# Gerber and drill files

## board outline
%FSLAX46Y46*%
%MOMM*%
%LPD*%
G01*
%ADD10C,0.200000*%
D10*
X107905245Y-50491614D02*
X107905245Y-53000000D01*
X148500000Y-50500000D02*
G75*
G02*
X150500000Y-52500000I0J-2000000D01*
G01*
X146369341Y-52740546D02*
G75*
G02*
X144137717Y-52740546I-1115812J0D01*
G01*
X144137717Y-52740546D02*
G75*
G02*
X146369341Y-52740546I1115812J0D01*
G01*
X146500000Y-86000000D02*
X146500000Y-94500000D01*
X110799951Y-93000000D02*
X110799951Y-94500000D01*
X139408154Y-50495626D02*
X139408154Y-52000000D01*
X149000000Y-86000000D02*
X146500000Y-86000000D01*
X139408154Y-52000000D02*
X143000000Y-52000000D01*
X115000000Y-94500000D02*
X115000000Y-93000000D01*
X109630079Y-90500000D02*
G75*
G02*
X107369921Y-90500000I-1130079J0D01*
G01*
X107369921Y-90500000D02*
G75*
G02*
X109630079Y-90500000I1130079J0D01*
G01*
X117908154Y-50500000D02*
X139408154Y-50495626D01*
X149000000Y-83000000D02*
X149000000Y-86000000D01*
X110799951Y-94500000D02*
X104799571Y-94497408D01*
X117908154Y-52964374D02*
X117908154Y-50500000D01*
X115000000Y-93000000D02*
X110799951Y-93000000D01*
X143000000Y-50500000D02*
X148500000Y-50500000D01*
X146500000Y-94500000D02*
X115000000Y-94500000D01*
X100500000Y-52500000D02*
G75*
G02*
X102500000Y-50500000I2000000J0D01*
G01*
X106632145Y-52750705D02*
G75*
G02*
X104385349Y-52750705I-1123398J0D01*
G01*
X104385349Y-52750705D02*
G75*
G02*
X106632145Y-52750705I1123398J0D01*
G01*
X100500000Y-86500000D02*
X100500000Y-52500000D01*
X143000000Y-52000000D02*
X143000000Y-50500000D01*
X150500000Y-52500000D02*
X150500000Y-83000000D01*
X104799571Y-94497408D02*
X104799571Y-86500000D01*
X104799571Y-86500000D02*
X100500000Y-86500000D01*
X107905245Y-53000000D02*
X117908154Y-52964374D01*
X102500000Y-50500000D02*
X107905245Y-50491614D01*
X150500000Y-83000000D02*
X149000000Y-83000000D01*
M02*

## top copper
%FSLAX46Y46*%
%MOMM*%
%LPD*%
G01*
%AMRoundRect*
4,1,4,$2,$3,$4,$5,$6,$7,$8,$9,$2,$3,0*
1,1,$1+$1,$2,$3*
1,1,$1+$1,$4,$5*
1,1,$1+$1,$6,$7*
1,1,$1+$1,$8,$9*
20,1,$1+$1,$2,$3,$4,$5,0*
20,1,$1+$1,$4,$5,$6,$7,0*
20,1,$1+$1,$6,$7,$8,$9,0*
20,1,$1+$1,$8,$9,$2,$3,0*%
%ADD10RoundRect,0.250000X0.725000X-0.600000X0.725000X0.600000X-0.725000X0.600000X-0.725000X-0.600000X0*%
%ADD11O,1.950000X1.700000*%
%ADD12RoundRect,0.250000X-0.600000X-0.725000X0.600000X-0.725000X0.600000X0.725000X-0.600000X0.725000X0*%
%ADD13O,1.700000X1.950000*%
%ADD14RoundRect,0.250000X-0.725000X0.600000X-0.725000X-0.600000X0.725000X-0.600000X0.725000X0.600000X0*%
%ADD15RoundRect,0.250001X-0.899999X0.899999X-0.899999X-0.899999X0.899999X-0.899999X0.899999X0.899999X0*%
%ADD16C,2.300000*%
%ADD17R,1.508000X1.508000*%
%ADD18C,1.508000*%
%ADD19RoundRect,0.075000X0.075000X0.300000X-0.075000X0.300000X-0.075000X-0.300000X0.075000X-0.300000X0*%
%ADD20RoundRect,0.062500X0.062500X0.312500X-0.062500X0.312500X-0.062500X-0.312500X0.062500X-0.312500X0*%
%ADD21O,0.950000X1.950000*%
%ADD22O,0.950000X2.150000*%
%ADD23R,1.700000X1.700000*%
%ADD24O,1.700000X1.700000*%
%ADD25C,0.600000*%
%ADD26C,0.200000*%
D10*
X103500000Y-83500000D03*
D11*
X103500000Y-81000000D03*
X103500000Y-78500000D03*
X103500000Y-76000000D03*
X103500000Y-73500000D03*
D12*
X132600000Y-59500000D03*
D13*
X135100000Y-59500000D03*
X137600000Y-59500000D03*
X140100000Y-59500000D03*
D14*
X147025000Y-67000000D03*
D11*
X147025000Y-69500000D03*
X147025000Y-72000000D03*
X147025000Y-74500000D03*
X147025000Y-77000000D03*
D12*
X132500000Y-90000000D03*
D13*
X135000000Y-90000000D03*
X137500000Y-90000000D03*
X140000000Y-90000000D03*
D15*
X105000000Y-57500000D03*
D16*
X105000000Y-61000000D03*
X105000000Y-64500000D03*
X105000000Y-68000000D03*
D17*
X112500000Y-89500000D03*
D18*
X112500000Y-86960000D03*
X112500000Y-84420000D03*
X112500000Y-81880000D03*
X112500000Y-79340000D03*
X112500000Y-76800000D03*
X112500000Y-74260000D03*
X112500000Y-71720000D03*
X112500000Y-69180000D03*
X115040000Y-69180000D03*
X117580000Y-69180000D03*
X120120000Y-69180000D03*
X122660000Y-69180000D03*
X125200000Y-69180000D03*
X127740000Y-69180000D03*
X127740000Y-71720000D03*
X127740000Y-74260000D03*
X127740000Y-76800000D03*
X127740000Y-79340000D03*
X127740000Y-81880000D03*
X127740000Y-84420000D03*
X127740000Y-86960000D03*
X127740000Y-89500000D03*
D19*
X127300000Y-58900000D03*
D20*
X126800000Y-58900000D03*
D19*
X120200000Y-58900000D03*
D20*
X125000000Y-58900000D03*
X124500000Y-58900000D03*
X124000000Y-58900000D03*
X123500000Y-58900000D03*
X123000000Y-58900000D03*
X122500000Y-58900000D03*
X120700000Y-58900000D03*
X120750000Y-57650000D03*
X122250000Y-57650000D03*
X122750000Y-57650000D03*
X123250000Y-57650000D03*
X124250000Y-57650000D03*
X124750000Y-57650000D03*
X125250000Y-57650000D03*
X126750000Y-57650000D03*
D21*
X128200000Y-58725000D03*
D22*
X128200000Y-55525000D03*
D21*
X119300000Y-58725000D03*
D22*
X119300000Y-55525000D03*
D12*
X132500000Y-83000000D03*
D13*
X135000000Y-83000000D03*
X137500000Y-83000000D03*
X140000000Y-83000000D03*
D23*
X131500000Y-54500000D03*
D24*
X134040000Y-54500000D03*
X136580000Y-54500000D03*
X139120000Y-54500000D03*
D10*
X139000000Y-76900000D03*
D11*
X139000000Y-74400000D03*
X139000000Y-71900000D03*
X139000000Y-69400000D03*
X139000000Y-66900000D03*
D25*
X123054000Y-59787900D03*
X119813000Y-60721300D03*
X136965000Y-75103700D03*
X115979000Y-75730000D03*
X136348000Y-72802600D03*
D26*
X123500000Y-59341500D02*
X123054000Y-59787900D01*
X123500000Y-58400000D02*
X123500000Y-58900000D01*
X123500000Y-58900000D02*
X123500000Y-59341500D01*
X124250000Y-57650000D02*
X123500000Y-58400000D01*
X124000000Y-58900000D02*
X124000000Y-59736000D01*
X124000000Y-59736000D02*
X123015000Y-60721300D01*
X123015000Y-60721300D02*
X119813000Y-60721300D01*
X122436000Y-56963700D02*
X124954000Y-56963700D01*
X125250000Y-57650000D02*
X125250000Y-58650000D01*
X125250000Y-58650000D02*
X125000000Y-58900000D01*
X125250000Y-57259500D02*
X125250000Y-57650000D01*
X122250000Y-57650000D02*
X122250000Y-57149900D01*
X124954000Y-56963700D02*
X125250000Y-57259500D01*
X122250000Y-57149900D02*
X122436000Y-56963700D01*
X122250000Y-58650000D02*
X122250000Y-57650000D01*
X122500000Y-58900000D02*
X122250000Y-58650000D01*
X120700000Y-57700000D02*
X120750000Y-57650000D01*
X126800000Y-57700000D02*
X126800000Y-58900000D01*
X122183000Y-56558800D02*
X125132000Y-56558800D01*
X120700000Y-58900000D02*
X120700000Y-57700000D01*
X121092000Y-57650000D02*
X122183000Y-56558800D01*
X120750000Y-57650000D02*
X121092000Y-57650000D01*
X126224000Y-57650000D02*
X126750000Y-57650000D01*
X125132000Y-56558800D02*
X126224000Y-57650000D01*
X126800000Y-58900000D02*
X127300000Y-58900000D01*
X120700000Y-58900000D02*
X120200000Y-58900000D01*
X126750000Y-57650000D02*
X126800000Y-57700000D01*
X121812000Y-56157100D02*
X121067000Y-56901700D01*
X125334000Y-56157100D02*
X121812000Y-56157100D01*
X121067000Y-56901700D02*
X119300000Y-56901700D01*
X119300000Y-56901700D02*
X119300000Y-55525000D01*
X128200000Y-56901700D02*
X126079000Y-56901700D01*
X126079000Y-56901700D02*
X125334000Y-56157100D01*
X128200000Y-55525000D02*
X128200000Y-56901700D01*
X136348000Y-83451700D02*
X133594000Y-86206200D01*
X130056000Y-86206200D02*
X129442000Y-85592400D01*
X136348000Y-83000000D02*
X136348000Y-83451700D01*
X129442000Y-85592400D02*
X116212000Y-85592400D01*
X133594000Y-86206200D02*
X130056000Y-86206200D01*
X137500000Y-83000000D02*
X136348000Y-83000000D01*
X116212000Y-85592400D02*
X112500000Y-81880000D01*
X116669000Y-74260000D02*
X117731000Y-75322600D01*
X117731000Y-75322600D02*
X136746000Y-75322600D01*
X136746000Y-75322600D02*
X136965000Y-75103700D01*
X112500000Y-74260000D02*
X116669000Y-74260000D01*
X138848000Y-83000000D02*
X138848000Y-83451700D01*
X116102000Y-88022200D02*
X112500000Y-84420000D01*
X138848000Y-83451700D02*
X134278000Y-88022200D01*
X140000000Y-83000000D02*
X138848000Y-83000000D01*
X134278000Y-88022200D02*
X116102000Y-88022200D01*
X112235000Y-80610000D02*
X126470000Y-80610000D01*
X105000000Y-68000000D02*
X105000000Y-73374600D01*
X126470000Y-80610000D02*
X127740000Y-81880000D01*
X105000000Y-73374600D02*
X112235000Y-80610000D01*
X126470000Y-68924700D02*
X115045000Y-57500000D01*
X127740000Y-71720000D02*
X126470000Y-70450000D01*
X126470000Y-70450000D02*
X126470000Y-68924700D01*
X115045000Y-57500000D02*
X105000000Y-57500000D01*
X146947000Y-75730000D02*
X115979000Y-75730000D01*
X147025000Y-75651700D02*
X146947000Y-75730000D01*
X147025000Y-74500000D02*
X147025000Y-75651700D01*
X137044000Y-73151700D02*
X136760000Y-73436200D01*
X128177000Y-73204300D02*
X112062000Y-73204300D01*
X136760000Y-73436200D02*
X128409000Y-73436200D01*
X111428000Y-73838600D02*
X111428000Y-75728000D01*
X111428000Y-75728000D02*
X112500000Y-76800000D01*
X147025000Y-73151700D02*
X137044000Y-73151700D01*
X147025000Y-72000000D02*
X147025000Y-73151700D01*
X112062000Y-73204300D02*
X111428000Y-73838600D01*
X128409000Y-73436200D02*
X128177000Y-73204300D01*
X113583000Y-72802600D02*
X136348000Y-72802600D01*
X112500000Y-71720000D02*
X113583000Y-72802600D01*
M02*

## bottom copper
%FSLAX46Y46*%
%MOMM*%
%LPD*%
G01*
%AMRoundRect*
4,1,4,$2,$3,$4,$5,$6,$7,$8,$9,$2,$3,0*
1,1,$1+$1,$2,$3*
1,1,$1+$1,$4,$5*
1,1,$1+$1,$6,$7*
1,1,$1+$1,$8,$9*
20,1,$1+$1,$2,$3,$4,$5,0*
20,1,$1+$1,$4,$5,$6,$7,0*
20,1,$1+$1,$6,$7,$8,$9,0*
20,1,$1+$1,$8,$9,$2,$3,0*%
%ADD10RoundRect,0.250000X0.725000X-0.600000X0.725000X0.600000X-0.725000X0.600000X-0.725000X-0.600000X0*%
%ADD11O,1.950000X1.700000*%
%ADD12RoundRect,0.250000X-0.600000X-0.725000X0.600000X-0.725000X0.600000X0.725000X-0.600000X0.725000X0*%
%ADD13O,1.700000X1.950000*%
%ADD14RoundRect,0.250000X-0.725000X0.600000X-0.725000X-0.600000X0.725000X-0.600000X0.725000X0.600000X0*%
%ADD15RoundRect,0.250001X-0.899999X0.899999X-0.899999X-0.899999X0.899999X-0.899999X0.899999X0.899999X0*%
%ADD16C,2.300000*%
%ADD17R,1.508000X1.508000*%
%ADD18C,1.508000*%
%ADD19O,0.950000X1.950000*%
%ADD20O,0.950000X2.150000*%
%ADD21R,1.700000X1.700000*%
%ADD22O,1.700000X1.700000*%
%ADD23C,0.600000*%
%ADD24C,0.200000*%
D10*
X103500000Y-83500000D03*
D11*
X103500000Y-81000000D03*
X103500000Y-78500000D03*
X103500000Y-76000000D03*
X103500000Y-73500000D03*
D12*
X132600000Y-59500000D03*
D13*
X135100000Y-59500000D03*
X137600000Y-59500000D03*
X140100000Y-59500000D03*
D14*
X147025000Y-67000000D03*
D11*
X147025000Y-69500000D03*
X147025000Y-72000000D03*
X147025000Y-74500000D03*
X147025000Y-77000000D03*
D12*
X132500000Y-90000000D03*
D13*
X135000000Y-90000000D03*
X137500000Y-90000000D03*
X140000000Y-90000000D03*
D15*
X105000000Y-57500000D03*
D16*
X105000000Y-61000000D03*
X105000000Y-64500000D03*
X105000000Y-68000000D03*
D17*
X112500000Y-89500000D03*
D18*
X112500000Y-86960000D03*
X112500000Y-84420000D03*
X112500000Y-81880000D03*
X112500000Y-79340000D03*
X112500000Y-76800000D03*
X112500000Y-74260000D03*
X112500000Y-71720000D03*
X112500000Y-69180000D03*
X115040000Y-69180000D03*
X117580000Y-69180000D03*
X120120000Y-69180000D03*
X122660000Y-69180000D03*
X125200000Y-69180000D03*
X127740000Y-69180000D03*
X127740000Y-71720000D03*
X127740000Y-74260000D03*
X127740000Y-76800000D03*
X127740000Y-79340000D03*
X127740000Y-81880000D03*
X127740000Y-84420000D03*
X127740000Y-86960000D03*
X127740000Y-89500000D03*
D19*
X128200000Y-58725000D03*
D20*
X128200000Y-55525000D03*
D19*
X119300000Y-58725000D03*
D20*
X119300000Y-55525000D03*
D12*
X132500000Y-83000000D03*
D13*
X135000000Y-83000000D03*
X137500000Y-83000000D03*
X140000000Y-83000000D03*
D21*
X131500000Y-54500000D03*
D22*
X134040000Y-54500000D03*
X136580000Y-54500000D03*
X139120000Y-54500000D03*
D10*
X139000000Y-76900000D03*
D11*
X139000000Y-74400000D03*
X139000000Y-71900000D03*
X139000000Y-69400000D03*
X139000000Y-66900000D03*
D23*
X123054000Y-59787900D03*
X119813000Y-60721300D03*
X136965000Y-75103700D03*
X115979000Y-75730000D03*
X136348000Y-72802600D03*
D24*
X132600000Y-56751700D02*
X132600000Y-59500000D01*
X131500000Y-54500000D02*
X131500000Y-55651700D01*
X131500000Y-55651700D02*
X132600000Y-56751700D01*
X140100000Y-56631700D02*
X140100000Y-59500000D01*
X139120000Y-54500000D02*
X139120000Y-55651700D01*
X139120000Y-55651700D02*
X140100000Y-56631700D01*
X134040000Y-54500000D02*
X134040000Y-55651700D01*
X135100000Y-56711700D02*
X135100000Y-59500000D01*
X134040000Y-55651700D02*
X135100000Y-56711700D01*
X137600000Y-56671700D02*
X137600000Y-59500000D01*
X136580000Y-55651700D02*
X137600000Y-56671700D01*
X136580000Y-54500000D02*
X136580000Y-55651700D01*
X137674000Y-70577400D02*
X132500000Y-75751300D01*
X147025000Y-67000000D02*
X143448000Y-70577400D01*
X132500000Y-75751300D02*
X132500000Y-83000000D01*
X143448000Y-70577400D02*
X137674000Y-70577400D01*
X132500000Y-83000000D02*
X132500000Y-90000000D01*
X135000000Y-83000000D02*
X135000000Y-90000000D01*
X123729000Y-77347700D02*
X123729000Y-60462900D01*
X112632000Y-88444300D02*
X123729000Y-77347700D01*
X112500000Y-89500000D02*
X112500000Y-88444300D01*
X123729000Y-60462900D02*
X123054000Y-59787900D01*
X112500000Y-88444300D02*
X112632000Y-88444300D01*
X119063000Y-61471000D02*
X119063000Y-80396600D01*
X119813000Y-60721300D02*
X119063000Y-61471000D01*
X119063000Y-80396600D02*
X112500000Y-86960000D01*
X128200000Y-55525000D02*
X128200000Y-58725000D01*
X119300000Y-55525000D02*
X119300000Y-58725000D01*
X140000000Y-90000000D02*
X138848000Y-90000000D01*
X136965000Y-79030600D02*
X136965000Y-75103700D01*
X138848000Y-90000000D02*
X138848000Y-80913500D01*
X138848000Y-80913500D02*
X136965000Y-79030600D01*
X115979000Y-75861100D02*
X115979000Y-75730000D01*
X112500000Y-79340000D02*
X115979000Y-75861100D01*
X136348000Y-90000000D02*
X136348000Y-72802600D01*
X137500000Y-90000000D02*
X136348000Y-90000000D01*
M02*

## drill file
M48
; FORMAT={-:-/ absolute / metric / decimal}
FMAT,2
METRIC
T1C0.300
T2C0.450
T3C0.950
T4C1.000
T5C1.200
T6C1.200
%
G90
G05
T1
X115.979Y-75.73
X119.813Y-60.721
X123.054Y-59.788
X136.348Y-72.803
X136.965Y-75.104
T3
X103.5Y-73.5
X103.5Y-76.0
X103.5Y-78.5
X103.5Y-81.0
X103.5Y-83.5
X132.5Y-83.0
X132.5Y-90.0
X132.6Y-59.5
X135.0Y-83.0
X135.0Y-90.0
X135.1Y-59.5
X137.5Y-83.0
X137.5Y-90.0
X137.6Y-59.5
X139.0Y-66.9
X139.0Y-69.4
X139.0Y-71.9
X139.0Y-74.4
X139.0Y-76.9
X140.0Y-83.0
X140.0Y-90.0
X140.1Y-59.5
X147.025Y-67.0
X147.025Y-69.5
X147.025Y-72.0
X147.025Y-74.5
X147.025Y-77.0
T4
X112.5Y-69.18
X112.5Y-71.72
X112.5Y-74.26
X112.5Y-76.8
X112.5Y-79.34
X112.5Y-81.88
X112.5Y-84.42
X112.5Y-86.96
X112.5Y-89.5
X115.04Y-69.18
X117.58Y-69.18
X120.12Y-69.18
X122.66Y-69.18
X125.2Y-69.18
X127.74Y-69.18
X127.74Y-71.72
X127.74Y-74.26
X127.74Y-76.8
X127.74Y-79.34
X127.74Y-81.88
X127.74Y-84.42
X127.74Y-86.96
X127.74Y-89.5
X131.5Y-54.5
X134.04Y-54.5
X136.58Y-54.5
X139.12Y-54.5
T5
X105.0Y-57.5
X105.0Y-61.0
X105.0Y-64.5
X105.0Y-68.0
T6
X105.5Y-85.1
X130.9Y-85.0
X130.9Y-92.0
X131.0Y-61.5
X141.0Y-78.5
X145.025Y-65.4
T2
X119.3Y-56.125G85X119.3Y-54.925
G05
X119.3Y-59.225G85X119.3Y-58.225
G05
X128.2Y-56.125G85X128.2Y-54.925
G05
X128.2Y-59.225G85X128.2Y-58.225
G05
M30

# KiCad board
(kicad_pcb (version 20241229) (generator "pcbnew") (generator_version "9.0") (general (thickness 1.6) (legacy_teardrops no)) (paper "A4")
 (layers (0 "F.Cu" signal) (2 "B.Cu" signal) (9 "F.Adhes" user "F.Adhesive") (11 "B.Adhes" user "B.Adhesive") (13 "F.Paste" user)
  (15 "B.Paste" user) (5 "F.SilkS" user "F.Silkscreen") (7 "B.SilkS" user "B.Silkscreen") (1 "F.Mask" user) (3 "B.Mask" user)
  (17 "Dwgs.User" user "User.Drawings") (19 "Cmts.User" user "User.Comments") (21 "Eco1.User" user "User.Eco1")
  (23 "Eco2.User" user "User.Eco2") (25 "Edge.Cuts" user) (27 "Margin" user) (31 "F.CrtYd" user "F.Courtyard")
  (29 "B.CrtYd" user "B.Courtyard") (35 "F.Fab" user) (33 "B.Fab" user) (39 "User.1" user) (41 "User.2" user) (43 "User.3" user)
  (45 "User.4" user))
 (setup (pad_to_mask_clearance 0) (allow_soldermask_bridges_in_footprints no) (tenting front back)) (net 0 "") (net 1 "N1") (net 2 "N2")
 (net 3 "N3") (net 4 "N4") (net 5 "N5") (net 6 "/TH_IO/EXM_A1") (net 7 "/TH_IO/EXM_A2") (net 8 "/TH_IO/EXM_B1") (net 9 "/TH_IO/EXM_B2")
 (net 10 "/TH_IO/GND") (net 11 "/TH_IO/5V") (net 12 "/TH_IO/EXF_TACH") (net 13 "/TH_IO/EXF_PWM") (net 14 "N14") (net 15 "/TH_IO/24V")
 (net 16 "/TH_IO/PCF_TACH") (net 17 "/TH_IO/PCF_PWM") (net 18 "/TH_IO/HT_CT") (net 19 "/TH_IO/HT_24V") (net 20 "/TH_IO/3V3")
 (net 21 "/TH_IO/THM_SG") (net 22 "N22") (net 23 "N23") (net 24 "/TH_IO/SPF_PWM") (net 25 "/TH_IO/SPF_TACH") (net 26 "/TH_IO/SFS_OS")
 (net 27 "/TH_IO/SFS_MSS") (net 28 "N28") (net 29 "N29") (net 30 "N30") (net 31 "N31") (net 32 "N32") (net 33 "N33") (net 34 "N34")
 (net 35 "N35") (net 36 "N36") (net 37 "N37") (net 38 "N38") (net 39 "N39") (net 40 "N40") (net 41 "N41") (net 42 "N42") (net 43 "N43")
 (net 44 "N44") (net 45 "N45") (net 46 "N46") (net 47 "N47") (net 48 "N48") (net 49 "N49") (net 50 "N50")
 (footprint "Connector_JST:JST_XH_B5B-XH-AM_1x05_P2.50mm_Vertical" (layer "F.Cu") (at 103.5 83.5 90)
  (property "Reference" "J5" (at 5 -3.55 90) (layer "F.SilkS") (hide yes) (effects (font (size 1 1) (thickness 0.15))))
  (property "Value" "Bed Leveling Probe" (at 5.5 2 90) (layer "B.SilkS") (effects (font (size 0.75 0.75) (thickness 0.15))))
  (pad "" np_thru_hole circle (at -1.6 2 90) (size 1.2 1.2) (drill 1.2) (layers "*.Cu" "*.Mask"))
  (pad "1" thru_hole roundrect (at 0 0 90) (size 1.7 1.95) (drill 0.95) (layers "*.Cu" "*.Mask") (remove_unused_layers no)
   (roundrect_rratio 0.147059) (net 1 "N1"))
  (pad "2" thru_hole oval (at 2.5 0 90) (size 1.7 1.95) (drill 0.95) (layers "*.Cu" "*.Mask") (remove_unused_layers no) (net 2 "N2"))
  (pad "3" thru_hole oval (at 5 0 90) (size 1.7 1.95) (drill 0.95) (layers "*.Cu" "*.Mask") (remove_unused_layers no) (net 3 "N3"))
  (pad "4" thru_hole oval (at 7.5 0 90) (size 1.7 1.95) (drill 0.95) (layers "*.Cu" "*.Mask") (remove_unused_layers no) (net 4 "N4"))
  (pad "5" thru_hole oval (at 10 0 90) (size 1.7 1.95) (drill 0.95) (layers "*.Cu" "*.Mask") (remove_unused_layers no) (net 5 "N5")))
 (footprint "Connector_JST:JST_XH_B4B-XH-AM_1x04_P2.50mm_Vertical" (layer "F.Cu") (at 132.6 59.5)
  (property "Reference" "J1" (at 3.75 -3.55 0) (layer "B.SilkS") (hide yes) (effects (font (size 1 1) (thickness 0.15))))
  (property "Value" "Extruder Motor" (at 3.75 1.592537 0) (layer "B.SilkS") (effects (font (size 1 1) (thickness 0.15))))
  (pad "" np_thru_hole circle (at -1.6 2) (size 1.2 1.2) (drill 1.2) (layers "*.Cu" "*.Mask"))
  (pad "1" thru_hole roundrect (at 0 0) (size 1.7 1.95) (drill 0.95) (layers "*.Cu" "*.Mask") (remove_unused_layers no)
   (roundrect_rratio 0.147059) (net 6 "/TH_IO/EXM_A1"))
  (pad "2" thru_hole oval (at 2.5 0) (size 1.7 1.95) (drill 0.95) (layers "*.Cu" "*.Mask") (remove_unused_layers no) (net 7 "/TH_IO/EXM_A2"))
  (pad "3" thru_hole oval (at 5 0) (size 1.7 1.95) (drill 0.95) (layers "*.Cu" "*.Mask") (remove_unused_layers no) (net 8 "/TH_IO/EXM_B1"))
  (pad "4" thru_hole oval (at 7.5 0) (size 1.7 1.95) (drill 0.95) (layers "*.Cu" "*.Mask") (remove_unused_layers no) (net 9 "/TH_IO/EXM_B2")))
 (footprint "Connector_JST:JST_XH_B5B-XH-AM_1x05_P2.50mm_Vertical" (layer "F.Cu") (at 147.025 67 -90)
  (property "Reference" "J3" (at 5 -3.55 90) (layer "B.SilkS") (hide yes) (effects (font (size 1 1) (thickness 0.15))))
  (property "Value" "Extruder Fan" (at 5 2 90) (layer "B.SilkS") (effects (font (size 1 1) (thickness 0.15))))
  (pad "" np_thru_hole circle (at -1.6 2 270) (size 1.2 1.2) (drill 1.2) (layers "*.Cu" "*.Mask"))
  (pad "1" thru_hole roundrect (at 0 0 270) (size 1.7 1.95) (drill 0.95) (layers "*.Cu" "*.Mask") (remove_unused_layers no)
   (roundrect_rratio 0.147059) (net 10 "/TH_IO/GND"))
  (pad "2" thru_hole oval (at 2.5 0 270) (size 1.7 1.95) (drill 0.95) (layers "*.Cu" "*.Mask") (remove_unused_layers no)
   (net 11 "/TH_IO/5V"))
  (pad "3" thru_hole oval (at 5 0 270) (size 1.7 1.95) (drill 0.95) (layers "*.Cu" "*.Mask") (remove_unused_layers no)
   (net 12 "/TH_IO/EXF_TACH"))
  (pad "4" thru_hole oval (at 7.5 0 270) (size 1.7 1.95) (drill 0.95) (layers "*.Cu" "*.Mask") (remove_unused_layers no)
   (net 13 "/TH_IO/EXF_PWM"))
  (pad "5" thru_hole oval (at 10 0 270) (size 1.7 1.95) (drill 0.95) (layers "*.Cu" "*.Mask") (remove_unused_layers no) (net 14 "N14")))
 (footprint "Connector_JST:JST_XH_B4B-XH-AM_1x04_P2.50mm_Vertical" (layer "F.Cu") (at 132.5 90)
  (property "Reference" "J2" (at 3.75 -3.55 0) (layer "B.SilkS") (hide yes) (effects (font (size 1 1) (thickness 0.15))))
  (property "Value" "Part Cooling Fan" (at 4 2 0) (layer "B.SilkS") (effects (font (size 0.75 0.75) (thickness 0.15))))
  (pad "" np_thru_hole circle (at -1.6 2) (size 1.2 1.2) (drill 1.2) (layers "*.Cu" "*.Mask"))
  (pad "1" thru_hole roundrect (at 0 0) (size 1.7 1.95) (drill 0.95) (layers "*.Cu" "*.Mask") (remove_unused_layers no)
   (roundrect_rratio 0.147059) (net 10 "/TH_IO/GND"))
  (pad "2" thru_hole oval (at 2.5 0) (size 1.7 1.95) (drill 0.95) (layers "*.Cu" "*.Mask") (remove_unused_layers no) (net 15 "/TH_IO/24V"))
  (pad "3" thru_hole oval (at 5 0) (size 1.7 1.95) (drill 0.95) (layers "*.Cu" "*.Mask") (remove_unused_layers no)
   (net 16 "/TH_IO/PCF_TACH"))
  (pad "4" thru_hole oval (at 7.5 0) (size 1.7 1.95) (drill 0.95) (layers "*.Cu" "*.Mask") (remove_unused_layers no)
   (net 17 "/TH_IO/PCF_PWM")))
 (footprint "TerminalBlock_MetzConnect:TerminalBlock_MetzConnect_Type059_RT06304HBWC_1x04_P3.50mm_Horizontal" (layer "F.Cu")
  (at 105 57.5 -90)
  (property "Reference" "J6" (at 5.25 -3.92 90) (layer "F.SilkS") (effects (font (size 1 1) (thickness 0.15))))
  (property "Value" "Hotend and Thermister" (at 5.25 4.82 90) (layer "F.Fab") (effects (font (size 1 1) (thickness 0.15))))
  (pad "1" thru_hole roundrect (at 0 0 270) (size 2.3 2.3) (drill 1.2) (layers "*.Cu" "*.Mask") (remove_unused_layers no)
   (roundrect_rratio 0.108696) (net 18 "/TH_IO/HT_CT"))
  (pad "2" thru_hole circle (at 3.5 0 270) (size 2.3 2.3) (drill 1.2) (layers "*.Cu" "*.Mask") (remove_unused_layers no)
   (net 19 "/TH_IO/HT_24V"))
  (pad "3" thru_hole circle (at 7 0 270) (size 2.3 2.3) (drill 1.2) (layers "*.Cu" "*.Mask") (remove_unused_layers no) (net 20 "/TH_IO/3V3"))
  (pad "4" thru_hole circle (at 10.5 0 270) (size 2.3 2.3) (drill 1.2) (layers "*.Cu" "*.Mask") (remove_unused_layers no)
   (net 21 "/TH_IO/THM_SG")))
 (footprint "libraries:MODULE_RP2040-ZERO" (layer "F.Cu") (at 120.12 79.34 180)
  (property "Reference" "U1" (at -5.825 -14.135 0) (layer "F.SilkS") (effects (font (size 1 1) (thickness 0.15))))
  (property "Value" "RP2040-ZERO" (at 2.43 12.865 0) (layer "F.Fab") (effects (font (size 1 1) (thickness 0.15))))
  (pad "1" thru_hole rect (at 7.62 -10.16 180) (size 1.508 1.508) (drill 1) (layers "*.Cu" "*.Mask") (remove_unused_layers no)
   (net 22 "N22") (solder_mask_margin 0.102))
  (pad "2" thru_hole circle (at 7.62 -7.62 180) (size 1.508 1.508) (drill 1) (layers "*.Cu" "*.Mask") (remove_unused_layers no)
   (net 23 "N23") (solder_mask_margin 0.102))
  (pad "3" thru_hole circle (at 7.62 -5.08 180) (size 1.508 1.508) (drill 1) (layers "*.Cu" "*.Mask") (remove_unused_layers no)
   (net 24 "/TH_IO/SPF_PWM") (solder_mask_margin 0.102))
  (pad "4" thru_hole circle (at 7.62 -2.54 180) (size 1.508 1.508) (drill 1) (layers "*.Cu" "*.Mask") (remove_unused_layers no)
   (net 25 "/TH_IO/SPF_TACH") (solder_mask_margin 0.102))
  (pad "5" thru_hole circle (at 7.62 0 180) (size 1.508 1.508) (drill 1) (layers "*.Cu" "*.Mask") (remove_unused_layers no)
   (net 13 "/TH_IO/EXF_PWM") (solder_mask_margin 0.102))
  (pad "6" thru_hole circle (at 7.62 2.54 180) (size 1.508 1.508) (drill 1) (layers "*.Cu" "*.Mask") (remove_unused_layers no)
   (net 12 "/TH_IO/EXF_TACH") (solder_mask_margin 0.102))
  (pad "7" thru_hole circle (at 7.62 5.08 180) (size 1.508 1.508) (drill 1) (layers "*.Cu" "*.Mask") (remove_unused_layers no)
   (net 17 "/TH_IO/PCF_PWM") (solder_mask_margin 0.102))
  (pad "8" thru_hole circle (at 7.62 7.62 180) (size 1.508 1.508) (drill 1) (layers "*.Cu" "*.Mask") (remove_unused_layers no)
   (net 16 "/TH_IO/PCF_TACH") (solder_mask_margin 0.102))
  (pad "9" thru_hole circle (at 7.62 10.16 180) (size 1.508 1.508) (drill 1) (layers "*.Cu" "*.Mask") (remove_unused_layers no)
   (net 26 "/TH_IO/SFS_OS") (solder_mask_margin 0.102))
  (pad "10" thru_hole circle (at 5.08 10.16 180) (size 1.508 1.508) (drill 1) (layers "*.Cu" "*.Mask") (remove_unused_layers no)
   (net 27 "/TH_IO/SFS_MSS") (solder_mask_margin 0.102))
  (pad "11" thru_hole circle (at 2.54 10.16 180) (size 1.508 1.508) (drill 1) (layers "*.Cu" "*.Mask") (remove_unused_layers no)
   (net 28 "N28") (solder_mask_margin 0.102))
  (pad "12" thru_hole circle (at 0 10.16 180) (size 1.508 1.508) (drill 1) (layers "*.Cu" "*.Mask") (remove_unused_layers no) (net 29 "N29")
   (solder_mask_margin 0.102))
  (pad "13" thru_hole circle (at -2.54 10.16 180) (size 1.508 1.508) (drill 1) (layers "*.Cu" "*.Mask") (remove_unused_layers no)
   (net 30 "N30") (solder_mask_margin 0.102))
  (pad "14" thru_hole circle (at -5.08 10.16 180) (size 1.508 1.508) (drill 1) (layers "*.Cu" "*.Mask") (remove_unused_layers no)
   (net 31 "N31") (solder_mask_margin 0.102))
  (pad "15" thru_hole circle (at -7.62 10.16 180) (size 1.508 1.508) (drill 1) (layers "*.Cu" "*.Mask") (remove_unused_layers no)
   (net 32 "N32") (solder_mask_margin 0.102))
  (pad "16" thru_hole circle (at -7.62 7.62 180) (size 1.508 1.508) (drill 1) (layers "*.Cu" "*.Mask") (remove_unused_layers no)
   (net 18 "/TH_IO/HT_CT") (solder_mask_margin 0.102))
  (pad "17" thru_hole circle (at -7.62 5.08 180) (size 1.508 1.508) (drill 1) (layers "*.Cu" "*.Mask") (remove_unused_layers no)
   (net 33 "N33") (solder_mask_margin 0.102))
  (pad "18" thru_hole circle (at -7.62 2.54 180) (size 1.508 1.508) (drill 1) (layers "*.Cu" "*.Mask") (remove_unused_layers no)
   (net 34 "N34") (solder_mask_margin 0.102))
  (pad "19" thru_hole circle (at -7.62 0 180) (size 1.508 1.508) (drill 1) (layers "*.Cu" "*.Mask") (remove_unused_layers no) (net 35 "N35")
   (solder_mask_margin 0.102))
  (pad "20" thru_hole circle (at -7.62 -2.54 180) (size 1.508 1.508) (drill 1) (layers "*.Cu" "*.Mask") (remove_unused_layers no)
   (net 21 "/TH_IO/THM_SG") (solder_mask_margin 0.102))
  (pad "21" thru_hole circle (at -7.62 -5.08 180) (size 1.508 1.508) (drill 1) (layers "*.Cu" "*.Mask") (remove_unused_layers no)
   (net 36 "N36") (solder_mask_margin 0.102))
  (pad "22" thru_hole circle (at -7.62 -7.62 180) (size 1.508 1.508) (drill 1) (layers "*.Cu" "*.Mask") (remove_unused_layers no)
   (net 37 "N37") (solder_mask_margin 0.102))
  (pad "23" thru_hole circle (at -7.62 -10.16 180) (size 1.508 1.508) (drill 1) (layers "*.Cu" "*.Mask") (remove_unused_layers no)
   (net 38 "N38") (solder_mask_margin 0.102)))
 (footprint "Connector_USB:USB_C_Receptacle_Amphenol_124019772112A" (layer "F.Cu") (at 123.75 55.7 180)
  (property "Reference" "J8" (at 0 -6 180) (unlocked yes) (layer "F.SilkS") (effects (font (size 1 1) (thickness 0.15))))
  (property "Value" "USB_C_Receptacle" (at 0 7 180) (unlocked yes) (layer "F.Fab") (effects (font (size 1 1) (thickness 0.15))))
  (pad "A1" smd roundrect (at -3.55 -3.2 180) (size 0.3 0.75) (layers "F.Cu" "F.Mask" "F.Paste") (roundrect_rratio 0.25) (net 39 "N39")
   (thermal_bridge_angle 45))
  (pad "A1" smd roundrect (at -3.05 -3.2 180) (size 0.25 0.75) (layers "F.Cu" "F.Mask" "F.Paste") (roundrect_rratio 0.25) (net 39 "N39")
   (thermal_bridge_angle 45))
  (pad "A1" smd roundrect (at 3.55 -3.2 180) (size 0.3 0.75) (layers "F.Cu" "F.Mask" "F.Paste") (roundrect_rratio 0.25) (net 39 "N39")
   (thermal_bridge_angle 45))
  (pad "A4" smd roundrect (at -1.25 -3.2 180) (size 0.25 0.75) (layers "F.Cu" "F.Mask" "F.Paste") (roundrect_rratio 0.25) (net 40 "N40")
   (thermal_bridge_angle 45))
  (pad "A5" smd roundrect (at -0.75 -3.2 180) (size 0.25 0.75) (layers "F.Cu" "F.Mask" "F.Paste") (roundrect_rratio 0.25) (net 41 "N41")
   (thermal_bridge_angle 45))
  (pad "A6" smd roundrect (at -0.25 -3.2 180) (size 0.25 0.75) (layers "F.Cu" "F.Mask" "F.Paste") (roundrect_rratio 0.25) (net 23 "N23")
   (thermal_bridge_angle 45))
  (pad "A7" smd roundrect (at 0.25 -3.2 180) (size 0.25 0.75) (layers "F.Cu" "F.Mask" "F.Paste") (roundrect_rratio 0.25) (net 22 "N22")
   (thermal_bridge_angle 45))
  (pad "A8" smd roundrect (at 0.75 -3.2 180) (size 0.25 0.75) (layers "F.Cu" "F.Mask" "F.Paste") (roundrect_rratio 0.25) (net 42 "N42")
   (thermal_bridge_angle 45))
  (pad "A9" smd roundrect (at 1.25 -3.2 180) (size 0.25 0.75) (layers "F.Cu" "F.Mask" "F.Paste") (roundrect_rratio 0.25) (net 40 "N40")
   (thermal_bridge_angle 45))
  (pad "A12" smd roundrect (at 3.05 -3.2 180) (size 0.25 0.75) (layers "F.Cu" "F.Mask" "F.Paste") (roundrect_rratio 0.25) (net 39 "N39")
   (thermal_bridge_angle 45))
  (pad "B1" smd roundrect (at 3 -1.95 180) (size 0.25 0.75) (layers "F.Cu" "F.Mask" "F.Paste") (roundrect_rratio 0.25) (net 39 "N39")
   (thermal_bridge_angle 45))
  (pad "B4" smd roundrect (at 1.5 -1.95 180) (size 0.25 0.75) (layers "F.Cu" "F.Mask" "F.Paste") (roundrect_rratio 0.25) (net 40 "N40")
   (thermal_bridge_angle 45))
  (pad "B5" smd roundrect (at 1 -1.95 180) (size 0.25 0.75) (layers "F.Cu" "F.Mask" "F.Paste") (roundrect_rratio 0.25) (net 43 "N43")
   (thermal_bridge_angle 45))
  (pad "B6" smd roundrect (at 0.5 -1.95 180) (size 0.25 0.75) (layers "F.Cu" "F.Mask" "F.Paste") (roundrect_rratio 0.25) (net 23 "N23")
   (thermal_bridge_angle 45))
  (pad "B7" smd roundrect (at -0.5 -1.95 180) (size 0.25 0.75) (layers "F.Cu" "F.Mask" "F.Paste") (roundrect_rratio 0.25) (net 22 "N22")
   (thermal_bridge_angle 45))
  (pad "B8" smd roundrect (at -1 -1.95 180) (size 0.25 0.75) (layers "F.Cu" "F.Mask" "F.Paste") (roundrect_rratio 0.25) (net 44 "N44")
   (thermal_bridge_angle 45))
  (pad "B9" smd roundrect (at -1.5 -1.95 180) (size 0.25 0.75) (layers "F.Cu" "F.Mask" "F.Paste") (roundrect_rratio 0.25) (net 40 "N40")
   (thermal_bridge_angle 45))
  (pad "B12" smd roundrect (at -3 -1.95 180) (size 0.25 0.75) (layers "F.Cu" "F.Mask" "F.Paste") (roundrect_rratio 0.25) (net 39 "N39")
   (thermal_bridge_angle 45))
  (pad "S1" thru_hole oval (at -4.45 -3.025 180) (size 0.95 1.95) (drill oval 0.45 1.45) (layers "*.Cu" "*.Mask") (remove_unused_layers no)
   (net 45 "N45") (thermal_bridge_angle 45))
  (pad "S1" thru_hole oval (at -4.45 0.175 180) (size 0.95 2.15) (drill oval 0.45 1.65) (layers "*.Cu" "*.Mask") (remove_unused_layers no)
   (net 45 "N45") (thermal_bridge_angle 45))
  (pad "S1" thru_hole oval (at 4.45 -3.025 180) (size 0.95 1.95) (drill oval 0.45 1.45) (layers "*.Cu" "*.Mask") (remove_unused_layers no)
   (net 45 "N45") (thermal_bridge_angle 45))
  (pad "S1" thru_hole oval (at 4.45 0.175 180) (size 0.95 2.15) (drill oval 0.45 1.65) (layers "*.Cu" "*.Mask") (remove_unused_layers no)
   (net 45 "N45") (thermal_bridge_angle 45)))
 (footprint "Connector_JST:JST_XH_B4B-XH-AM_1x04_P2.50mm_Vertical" (layer "F.Cu") (at 132.5 83)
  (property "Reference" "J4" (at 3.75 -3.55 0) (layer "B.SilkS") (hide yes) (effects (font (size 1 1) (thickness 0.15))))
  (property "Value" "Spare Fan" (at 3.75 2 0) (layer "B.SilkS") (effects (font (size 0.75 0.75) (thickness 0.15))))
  (pad "" np_thru_hole circle (at -1.6 2) (size 1.2 1.2) (drill 1.2) (layers "*.Cu" "*.Mask"))
  (pad "1" thru_hole roundrect (at 0 0) (size 1.7 1.95) (drill 0.95) (layers "*.Cu" "*.Mask") (remove_unused_layers no)
   (roundrect_rratio 0.147059) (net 10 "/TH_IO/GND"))
  (pad "2" thru_hole oval (at 2.5 0) (size 1.7 1.95) (drill 0.95) (layers "*.Cu" "*.Mask") (remove_unused_layers no) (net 15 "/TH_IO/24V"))
  (pad "3" thru_hole oval (at 5 0) (size 1.7 1.95) (drill 0.95) (layers "*.Cu" "*.Mask") (remove_unused_layers no)
   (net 25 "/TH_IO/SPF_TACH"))
  (pad "4" thru_hole oval (at 7.5 0) (size 1.7 1.95) (drill 0.95) (layers "*.Cu" "*.Mask") (remove_unused_layers no)
   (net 24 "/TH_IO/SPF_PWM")))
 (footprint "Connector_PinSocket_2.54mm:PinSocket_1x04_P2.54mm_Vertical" (layer "F.Cu") (at 131.5 54.5 90)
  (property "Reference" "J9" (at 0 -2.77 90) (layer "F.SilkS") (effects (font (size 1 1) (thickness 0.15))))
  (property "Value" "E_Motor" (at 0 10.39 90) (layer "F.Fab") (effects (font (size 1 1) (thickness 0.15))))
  (pad "1" thru_hole rect (at 0 0 90) (size 1.7 1.7) (drill 1) (layers "*.Cu" "*.Mask") (remove_unused_layers no) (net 6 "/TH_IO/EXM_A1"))
  (pad "2" thru_hole oval (at 0 2.54 90) (size 1.7 1.7) (drill 1) (layers "*.Cu" "*.Mask") (remove_unused_layers no) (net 7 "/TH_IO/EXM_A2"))
  (pad "3" thru_hole oval (at 0 5.08 90) (size 1.7 1.7) (drill 1) (layers "*.Cu" "*.Mask") (remove_unused_layers no) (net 8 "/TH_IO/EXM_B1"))
  (pad "4" thru_hole oval (at 0 7.62 90) (size 1.7 1.7) (drill 1) (layers "*.Cu" "*.Mask") (remove_unused_layers no) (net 9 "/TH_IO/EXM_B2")))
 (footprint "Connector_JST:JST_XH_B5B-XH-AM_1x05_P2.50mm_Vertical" (layer "F.Cu") (at 139 76.9 90)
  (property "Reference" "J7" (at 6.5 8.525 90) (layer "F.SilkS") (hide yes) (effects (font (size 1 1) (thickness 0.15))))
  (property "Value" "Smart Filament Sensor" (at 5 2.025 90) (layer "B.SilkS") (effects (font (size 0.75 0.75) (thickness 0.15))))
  (pad "" np_thru_hole circle (at -1.6 2 90) (size 1.2 1.2) (drill 1.2) (layers "*.Cu" "*.Mask"))
  (pad "1" thru_hole roundrect (at 0 0 90) (size 1.7 1.95) (drill 0.95) (layers "*.Cu" "*.Mask") (remove_unused_layers no)
   (roundrect_rratio 0.147059) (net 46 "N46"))
  (pad "2" thru_hole oval (at 2.5 0 90) (size 1.7 1.95) (drill 0.95) (layers "*.Cu" "*.Mask") (remove_unused_layers no) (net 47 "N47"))
  (pad "3" thru_hole oval (at 5 0 90) (size 1.7 1.95) (drill 0.95) (layers "*.Cu" "*.Mask") (remove_unused_layers no) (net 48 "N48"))
  (pad "4" thru_hole oval (at 7.5 0 90) (size 1.7 1.95) (drill 0.95) (layers "*.Cu" "*.Mask") (remove_unused_layers no) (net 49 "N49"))
  (pad "5" thru_hole oval (at 10 0 90) (size 1.7 1.95) (drill 0.95) (layers "*.Cu" "*.Mask") (remove_unused_layers no) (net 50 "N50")))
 (gr_line (start 107.905245 50.491614) (end 107.905245 53) (stroke (width 0.2) (type solid)) (layer "Edge.Cuts"))
 (gr_arc (start 148.5 50.5) (mid 149.914214 51.085786) (end 150.5 52.5) (stroke (width 0.2) (type solid)) (layer "Edge.Cuts"))
 (gr_circle (center 145.253529 52.740546) (end 144.138266 52.775535) (stroke (width 0.2) (type solid)) (fill no) (layer "Edge.Cuts"))
 (gr_line (start 146.5 86) (end 146.5 94.5) (stroke (width 0.2) (type solid)) (layer "Edge.Cuts"))
 (gr_line (start 110.799951 93) (end 110.799951 94.5) (stroke (width 0.2) (type solid)) (layer "Edge.Cuts"))
 (gr_line (start 139.408154 50.495626) (end 139.408154 52) (stroke (width 0.2) (type solid)) (layer "Edge.Cuts"))
 (gr_line (start 149 86) (end 146.5 86) (stroke (width 0.2) (type solid)) (layer "Edge.Cuts"))
 (gr_line (start 139.408154 52) (end 143 52) (stroke (width 0.2) (type solid)) (layer "Edge.Cuts"))
 (gr_line (start 115 94.5) (end 115 93) (stroke (width 0.2) (type solid)) (layer "Edge.Cuts"))
 (gr_circle (center 108.5 90.5) (end 107.370204 90.474714) (stroke (width 0.2) (type solid)) (fill no) (layer "Edge.Cuts"))
 (gr_line (start 117.908154 50.5) (end 139.408154 50.495626) (stroke (width 0.2) (type solid)) (layer "Edge.Cuts"))
 (gr_line (start 149 83) (end 149 86) (stroke (width 0.2) (type solid)) (layer "Edge.Cuts"))
 (gr_line (start 110.799951 94.5) (end 104.799571 94.497408) (stroke (width 0.2) (type solid)) (layer "Edge.Cuts"))
 (gr_line (start 117.908154 52.964374) (end 117.908154 50.5) (stroke (width 0.2) (type solid)) (layer "Edge.Cuts"))
 (gr_line (start 115 93) (end 110.799951 93) (stroke (width 0.2) (type solid)) (layer "Edge.Cuts"))
 (gr_line (start 143 50.5) (end 148.5 50.5) (stroke (width 0.2) (type solid)) (layer "Edge.Cuts"))
 (gr_line (start 146.5 94.5) (end 115 94.5) (stroke (width 0.2) (type solid)) (layer "Edge.Cuts"))
 (gr_arc (start 100.5 52.5) (mid 101.085786 51.085786) (end 102.5 50.5) (stroke (width 0.2) (type solid)) (layer "Edge.Cuts"))
 (gr_circle (center 105.508747 52.750705) (end 104.38911 52.842551) (stroke (width 0.2) (type solid)) (fill no) (layer "Edge.Cuts"))
 (gr_line (start 100.5 86.5) (end 100.5 52.5) (stroke (width 0.2) (type solid)) (layer "Edge.Cuts"))
 (gr_line (start 143 52) (end 143 50.5) (stroke (width 0.2) (type solid)) (layer "Edge.Cuts"))
 (gr_line (start 150.5 52.5) (end 150.5 83) (stroke (width 0.2) (type solid)) (layer "Edge.Cuts"))
 (gr_line (start 104.799571 94.497408) (end 104.799571 86.5) (stroke (width 0.2) (type solid)) (layer "Edge.Cuts"))
 (gr_line (start 104.799571 86.5) (end 100.5 86.5) (stroke (width 0.2) (type solid)) (layer "Edge.Cuts"))
 (gr_line (start 107.905245 53) (end 117.908154 52.964374) (stroke (width 0.2) (type solid)) (layer "Edge.Cuts"))
 (gr_line (start 102.5 50.5) (end 107.905245 50.491614) (stroke (width 0.2) (type solid)) (layer "Edge.Cuts"))
 (gr_line (start 150.5 83) (end 149 83) (stroke (width 0.2) (type solid)) (layer "Edge.Cuts"))
 (segment (start 132.6 56.7517) (end 132.6 59.5) (width 0.2) (layer "B.Cu") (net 6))
 (segment (start 131.5 54.5) (end 131.5 55.6517) (width 0.2) (layer "B.Cu") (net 6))
 (segment (start 131.5 55.6517) (end 132.6 56.7517) (width 0.2) (layer "B.Cu") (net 6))
 (segment (start 140.1 56.6317) (end 140.1 59.5) (width 0.2) (layer "B.Cu") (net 9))
 (segment (start 139.12 54.5) (end 139.12 55.6517) (width 0.2) (layer "B.Cu") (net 9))
 (segment (start 139.12 55.6517) (end 140.1 56.6317) (width 0.2) (layer "B.Cu") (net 9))
 (segment (start 134.04 54.5) (end 134.04 55.6517) (width 0.2) (layer "B.Cu") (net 7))
 (segment (start 135.1 56.7117) (end 135.1 59.5) (width 0.2) (layer "B.Cu") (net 7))
 (segment (start 134.04 55.6517) (end 135.1 56.7117) (width 0.2) (layer "B.Cu") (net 7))
 (segment (start 137.6 56.6717) (end 137.6 59.5) (width 0.2) (layer "B.Cu") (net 8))
 (segment (start 136.58 55.6517) (end 137.6 56.6717) (width 0.2) (layer "B.Cu") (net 8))
 (segment (start 136.58 54.5) (end 136.58 55.6517) (width 0.2) (layer "B.Cu") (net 8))
 (segment (start 137.674 70.5774) (end 132.5 75.7513) (width 0.2) (layer "B.Cu") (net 10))
 (segment (start 147.025 67) (end 143.448 70.5774) (width 0.2) (layer "B.Cu") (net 10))
 (segment (start 132.5 75.7513) (end 132.5 83) (width 0.2) (layer "B.Cu") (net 10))
 (segment (start 143.448 70.5774) (end 137.674 70.5774) (width 0.2) (layer "B.Cu") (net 10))
 (segment (start 132.5 83) (end 132.5 90) (width 0.2) (layer "B.Cu") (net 10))
 (segment (start 135 83) (end 135 90) (width 0.2) (layer "B.Cu") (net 15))
 (segment (start 123.5 59.3415) (end 123.054 59.7879) (width 0.2) (layer "F.Cu") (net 22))
 (segment (start 123.5 58.4) (end 123.5 58.9) (width 0.2) (layer "F.Cu") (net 22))
 (segment (start 123.5 58.9) (end 123.5 59.3415) (width 0.2) (layer "F.Cu") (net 22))
 (segment (start 124.25 57.65) (end 123.5 58.4) (width 0.2) (layer "F.Cu") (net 22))
 (via (at 123.054 59.7879) (size 0.6) (drill 0.3) (layers "F.Cu" "B.Cu") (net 22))
 (segment (start 123.729 77.3477) (end 123.729 60.4629) (width 0.2) (layer "B.Cu") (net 22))
 (segment (start 112.632 88.4443) (end 123.729 77.3477) (width 0.2) (layer "B.Cu") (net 22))
 (segment (start 112.5 89.5) (end 112.5 88.4443) (width 0.2) (layer "B.Cu") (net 22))
 (segment (start 123.729 60.4629) (end 123.054 59.7879) (width 0.2) (layer "B.Cu") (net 22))
 (segment (start 112.5 88.4443) (end 112.632 88.4443) (width 0.2) (layer "B.Cu") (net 22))
 (segment (start 124 58.9) (end 124 59.736) (width 0.2) (layer "F.Cu") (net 23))
 (segment (start 124 59.736) (end 123.015 60.7213) (width 0.2) (layer "F.Cu") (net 23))
 (segment (start 123.015 60.7213) (end 119.813 60.7213) (width 0.2) (layer "F.Cu") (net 23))
 (via (at 119.813 60.7213) (size 0.6) (drill 0.3) (layers "F.Cu" "B.Cu") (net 23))
 (segment (start 119.063 61.471) (end 119.063 80.3966) (width 0.2) (layer "B.Cu") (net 23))
 (segment (start 119.813 60.7213) (end 119.063 61.471) (width 0.2) (layer "B.Cu") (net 23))
 (segment (start 119.063 80.3966) (end 112.5 86.96) (width 0.2) (layer "B.Cu") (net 23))
 (segment (start 122.436 56.9637) (end 124.954 56.9637) (width 0.2) (layer "F.Cu") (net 40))
 (segment (start 125.25 57.65) (end 125.25 58.65) (width 0.2) (layer "F.Cu") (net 40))
 (segment (start 125.25 58.65) (end 125 58.9) (width 0.2) (layer "F.Cu") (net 40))
 (segment (start 125.25 57.2595) (end 125.25 57.65) (width 0.2) (layer "F.Cu") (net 40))
 (segment (start 122.25 57.65) (end 122.25 57.1499) (width 0.2) (layer "F.Cu") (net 40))
 (segment (start 124.954 56.9637) (end 125.25 57.2595) (width 0.2) (layer "F.Cu") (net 40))
 (segment (start 122.25 57.1499) (end 122.436 56.9637) (width 0.2) (layer "F.Cu") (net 40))
 (segment (start 122.25 58.65) (end 122.25 57.65) (width 0.2) (layer "F.Cu") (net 40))
 (segment (start 122.5 58.9) (end 122.25 58.65) (width 0.2) (layer "F.Cu") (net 40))
 (segment (start 120.7 57.7) (end 120.75 57.65) (width 0.2) (layer "F.Cu") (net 39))
 (segment (start 126.8 57.7) (end 126.8 58.9) (width 0.2) (layer "F.Cu") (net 39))
 (segment (start 122.183 56.5588) (end 125.132 56.5588) (width 0.2) (layer "F.Cu") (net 39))
 (segment (start 120.7 58.9) (end 120.7 57.7) (width 0.2) (layer "F.Cu") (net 39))
 (segment (start 121.092 57.65) (end 122.183 56.5588) (width 0.2) (layer "F.Cu") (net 39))
 (segment (start 120.75 57.65) (end 121.092 57.65) (width 0.2) (layer "F.Cu") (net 39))
 (segment (start 126.224 57.65) (end 126.75 57.65) (width 0.2) (layer "F.Cu") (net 39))
 (segment (start 125.132 56.5588) (end 126.224 57.65) (width 0.2) (layer "F.Cu") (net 39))
 (segment (start 126.8 58.9) (end 127.3 58.9) (width 0.2) (layer "F.Cu") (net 39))
 (segment (start 120.7 58.9) (end 120.2 58.9) (width 0.2) (layer "F.Cu") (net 39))
 (segment (start 126.75 57.65) (end 126.8 57.7) (width 0.2) (layer "F.Cu") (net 39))
 (segment (start 121.812 56.1571) (end 121.067 56.9017) (width 0.2) (layer "F.Cu") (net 45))
 (segment (start 125.334 56.1571) (end 121.812 56.1571) (width 0.2) (layer "F.Cu") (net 45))
 (segment (start 121.067 56.9017) (end 119.3 56.9017) (width 0.2) (layer "F.Cu") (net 45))
 (segment (start 119.3 56.9017) (end 119.3 55.525) (width 0.2) (layer "F.Cu") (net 45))
 (segment (start 128.2 56.9017) (end 126.079 56.9017) (width 0.2) (layer "F.Cu") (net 45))
 (segment (start 126.079 56.9017) (end 125.334 56.1571) (width 0.2) (layer "F.Cu") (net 45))
 (segment (start 128.2 55.525) (end 128.2 56.9017) (width 0.2) (layer "F.Cu") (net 45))
 (segment (start 128.2 55.525) (end 128.2 58.725) (width 0.2) (layer "B.Cu") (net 45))
 (segment (start 119.3 55.525) (end 119.3 58.725) (width 0.2) (layer "B.Cu") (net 45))
 (segment (start 136.348 83.4517) (end 133.594 86.2062) (width 0.2) (layer "F.Cu") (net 25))
 (segment (start 130.056 86.2062) (end 129.442 85.5924) (width 0.2) (layer "F.Cu") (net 25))
 (segment (start 136.348 83) (end 136.348 83.4517) (width 0.2) (layer "F.Cu") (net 25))
 (segment (start 129.442 85.5924) (end 116.212 85.5924) (width 0.2) (layer "F.Cu") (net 25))
 (segment (start 133.594 86.2062) (end 130.056 86.2062) (width 0.2) (layer "F.Cu") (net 25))
 (segment (start 137.5 83) (end 136.348 83) (width 0.2) (layer "F.Cu") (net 25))
 (segment (start 116.212 85.5924) (end 112.5 81.88) (width 0.2) (layer "F.Cu") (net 25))
 (segment (start 116.669 74.26) (end 117.731 75.3226) (width 0.2) (layer "F.Cu") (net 17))
 (segment (start 117.731 75.3226) (end 136.746 75.3226) (width 0.2) (layer "F.Cu") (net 17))
 (segment (start 136.746 75.3226) (end 136.965 75.1037) (width 0.2) (layer "F.Cu") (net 17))
 (segment (start 112.5 74.26) (end 116.669 74.26) (width 0.2) (layer "F.Cu") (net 17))
 (via (at 136.965 75.1037) (size 0.6) (drill 0.3) (layers "F.Cu" "B.Cu") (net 17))
 (segment (start 140 90) (end 138.848 90) (width 0.2) (layer "B.Cu") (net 17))
 (segment (start 136.965 79.0306) (end 136.965 75.1037) (width 0.2) (layer "B.Cu") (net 17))
 (segment (start 138.848 90) (end 138.848 80.9135) (width 0.2) (layer "B.Cu") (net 17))
 (segment (start 138.848 80.9135) (end 136.965 79.0306) (width 0.2) (layer "B.Cu") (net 17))
 (segment (start 138.848 83) (end 138.848 83.4517) (width 0.2) (layer "F.Cu") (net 24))
 (segment (start 116.102 88.0222) (end 112.5 84.42) (width 0.2) (layer "F.Cu") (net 24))
 (segment (start 138.848 83.4517) (end 134.278 88.0222) (width 0.2) (layer "F.Cu") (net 24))
 (segment (start 140 83) (end 138.848 83) (width 0.2) (layer "F.Cu") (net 24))
 (segment (start 134.278 88.0222) (end 116.102 88.0222) (width 0.2) (layer "F.Cu") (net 24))
 (segment (start 112.235 80.61) (end 126.47 80.61) (width 0.2) (layer "F.Cu") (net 21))
 (segment (start 105 68) (end 105 73.3746) (width 0.2) (layer "F.Cu") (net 21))
 (segment (start 126.47 80.61) (end 127.74 81.88) (width 0.2) (layer "F.Cu") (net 21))
 (segment (start 105 73.3746) (end 112.235 80.61) (width 0.2) (layer "F.Cu") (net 21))
 (segment (start 126.47 68.9247) (end 115.045 57.5) (width 0.2) (layer "F.Cu") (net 18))
 (segment (start 127.74 71.72) (end 126.47 70.45) (width 0.2) (layer "F.Cu") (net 18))
 (segment (start 126.47 70.45) (end 126.47 68.9247) (width 0.2) (layer "F.Cu") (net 18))
 (segment (start 115.045 57.5) (end 105 57.5) (width 0.2) (layer "F.Cu") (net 18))
 (segment (start 146.947 75.73) (end 115.979 75.73) (width 0.2) (layer "F.Cu") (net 13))
 (segment (start 147.025 75.6517) (end 146.947 75.73) (width 0.2) (layer "F.Cu") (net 13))
 (segment (start 147.025 74.5) (end 147.025 75.6517) (width 0.2) (layer "F.Cu") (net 13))
 (via (at 115.979 75.73) (size 0.6) (drill 0.3) (layers "F.Cu" "B.Cu") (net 13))
 (segment (start 115.979 75.8611) (end 115.979 75.73) (width 0.2) (layer "B.Cu") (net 13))
 (segment (start 112.5 79.34) (end 115.979 75.8611) (width 0.2) (layer "B.Cu") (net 13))
 (segment (start 137.044 73.1517) (end 136.76 73.4362) (width 0.2) (layer "F.Cu") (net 12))
 (segment (start 128.177 73.2043) (end 112.062 73.2043) (width 0.2) (layer "F.Cu") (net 12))
 (segment (start 136.76 73.4362) (end 128.409 73.4362) (width 0.2) (layer "F.Cu") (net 12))
 (segment (start 111.428 73.8386) (end 111.428 75.728) (width 0.2) (layer "F.Cu") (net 12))
 (segment (start 111.428 75.728) (end 112.5 76.8) (width 0.2) (layer "F.Cu") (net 12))
 (segment (start 147.025 73.1517) (end 137.044 73.1517) (width 0.2) (layer "F.Cu") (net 12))
 (segment (start 147.025 72) (end 147.025 73.1517) (width 0.2) (layer "F.Cu") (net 12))
 (segment (start 112.062 73.2043) (end 111.428 73.8386) (width 0.2) (layer "F.Cu") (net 12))
 (segment (start 128.409 73.4362) (end 128.177 73.2043) (width 0.2) (layer "F.Cu") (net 12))
 (segment (start 113.583 72.8026) (end 136.348 72.8026) (width 0.2) (layer "F.Cu") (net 16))
 (segment (start 112.5 71.72) (end 113.583 72.8026) (width 0.2) (layer "F.Cu") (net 16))
 (via (at 136.348 72.8026) (size 0.6) (drill 0.3) (layers "F.Cu" "B.Cu") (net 16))
 (segment (start 136.348 90) (end 136.348 72.8026) (width 0.2) (layer "B.Cu") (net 16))
 (segment (start 137.5 90) (end 136.348 90) (width 0.2) (layer "B.Cu") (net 16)))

